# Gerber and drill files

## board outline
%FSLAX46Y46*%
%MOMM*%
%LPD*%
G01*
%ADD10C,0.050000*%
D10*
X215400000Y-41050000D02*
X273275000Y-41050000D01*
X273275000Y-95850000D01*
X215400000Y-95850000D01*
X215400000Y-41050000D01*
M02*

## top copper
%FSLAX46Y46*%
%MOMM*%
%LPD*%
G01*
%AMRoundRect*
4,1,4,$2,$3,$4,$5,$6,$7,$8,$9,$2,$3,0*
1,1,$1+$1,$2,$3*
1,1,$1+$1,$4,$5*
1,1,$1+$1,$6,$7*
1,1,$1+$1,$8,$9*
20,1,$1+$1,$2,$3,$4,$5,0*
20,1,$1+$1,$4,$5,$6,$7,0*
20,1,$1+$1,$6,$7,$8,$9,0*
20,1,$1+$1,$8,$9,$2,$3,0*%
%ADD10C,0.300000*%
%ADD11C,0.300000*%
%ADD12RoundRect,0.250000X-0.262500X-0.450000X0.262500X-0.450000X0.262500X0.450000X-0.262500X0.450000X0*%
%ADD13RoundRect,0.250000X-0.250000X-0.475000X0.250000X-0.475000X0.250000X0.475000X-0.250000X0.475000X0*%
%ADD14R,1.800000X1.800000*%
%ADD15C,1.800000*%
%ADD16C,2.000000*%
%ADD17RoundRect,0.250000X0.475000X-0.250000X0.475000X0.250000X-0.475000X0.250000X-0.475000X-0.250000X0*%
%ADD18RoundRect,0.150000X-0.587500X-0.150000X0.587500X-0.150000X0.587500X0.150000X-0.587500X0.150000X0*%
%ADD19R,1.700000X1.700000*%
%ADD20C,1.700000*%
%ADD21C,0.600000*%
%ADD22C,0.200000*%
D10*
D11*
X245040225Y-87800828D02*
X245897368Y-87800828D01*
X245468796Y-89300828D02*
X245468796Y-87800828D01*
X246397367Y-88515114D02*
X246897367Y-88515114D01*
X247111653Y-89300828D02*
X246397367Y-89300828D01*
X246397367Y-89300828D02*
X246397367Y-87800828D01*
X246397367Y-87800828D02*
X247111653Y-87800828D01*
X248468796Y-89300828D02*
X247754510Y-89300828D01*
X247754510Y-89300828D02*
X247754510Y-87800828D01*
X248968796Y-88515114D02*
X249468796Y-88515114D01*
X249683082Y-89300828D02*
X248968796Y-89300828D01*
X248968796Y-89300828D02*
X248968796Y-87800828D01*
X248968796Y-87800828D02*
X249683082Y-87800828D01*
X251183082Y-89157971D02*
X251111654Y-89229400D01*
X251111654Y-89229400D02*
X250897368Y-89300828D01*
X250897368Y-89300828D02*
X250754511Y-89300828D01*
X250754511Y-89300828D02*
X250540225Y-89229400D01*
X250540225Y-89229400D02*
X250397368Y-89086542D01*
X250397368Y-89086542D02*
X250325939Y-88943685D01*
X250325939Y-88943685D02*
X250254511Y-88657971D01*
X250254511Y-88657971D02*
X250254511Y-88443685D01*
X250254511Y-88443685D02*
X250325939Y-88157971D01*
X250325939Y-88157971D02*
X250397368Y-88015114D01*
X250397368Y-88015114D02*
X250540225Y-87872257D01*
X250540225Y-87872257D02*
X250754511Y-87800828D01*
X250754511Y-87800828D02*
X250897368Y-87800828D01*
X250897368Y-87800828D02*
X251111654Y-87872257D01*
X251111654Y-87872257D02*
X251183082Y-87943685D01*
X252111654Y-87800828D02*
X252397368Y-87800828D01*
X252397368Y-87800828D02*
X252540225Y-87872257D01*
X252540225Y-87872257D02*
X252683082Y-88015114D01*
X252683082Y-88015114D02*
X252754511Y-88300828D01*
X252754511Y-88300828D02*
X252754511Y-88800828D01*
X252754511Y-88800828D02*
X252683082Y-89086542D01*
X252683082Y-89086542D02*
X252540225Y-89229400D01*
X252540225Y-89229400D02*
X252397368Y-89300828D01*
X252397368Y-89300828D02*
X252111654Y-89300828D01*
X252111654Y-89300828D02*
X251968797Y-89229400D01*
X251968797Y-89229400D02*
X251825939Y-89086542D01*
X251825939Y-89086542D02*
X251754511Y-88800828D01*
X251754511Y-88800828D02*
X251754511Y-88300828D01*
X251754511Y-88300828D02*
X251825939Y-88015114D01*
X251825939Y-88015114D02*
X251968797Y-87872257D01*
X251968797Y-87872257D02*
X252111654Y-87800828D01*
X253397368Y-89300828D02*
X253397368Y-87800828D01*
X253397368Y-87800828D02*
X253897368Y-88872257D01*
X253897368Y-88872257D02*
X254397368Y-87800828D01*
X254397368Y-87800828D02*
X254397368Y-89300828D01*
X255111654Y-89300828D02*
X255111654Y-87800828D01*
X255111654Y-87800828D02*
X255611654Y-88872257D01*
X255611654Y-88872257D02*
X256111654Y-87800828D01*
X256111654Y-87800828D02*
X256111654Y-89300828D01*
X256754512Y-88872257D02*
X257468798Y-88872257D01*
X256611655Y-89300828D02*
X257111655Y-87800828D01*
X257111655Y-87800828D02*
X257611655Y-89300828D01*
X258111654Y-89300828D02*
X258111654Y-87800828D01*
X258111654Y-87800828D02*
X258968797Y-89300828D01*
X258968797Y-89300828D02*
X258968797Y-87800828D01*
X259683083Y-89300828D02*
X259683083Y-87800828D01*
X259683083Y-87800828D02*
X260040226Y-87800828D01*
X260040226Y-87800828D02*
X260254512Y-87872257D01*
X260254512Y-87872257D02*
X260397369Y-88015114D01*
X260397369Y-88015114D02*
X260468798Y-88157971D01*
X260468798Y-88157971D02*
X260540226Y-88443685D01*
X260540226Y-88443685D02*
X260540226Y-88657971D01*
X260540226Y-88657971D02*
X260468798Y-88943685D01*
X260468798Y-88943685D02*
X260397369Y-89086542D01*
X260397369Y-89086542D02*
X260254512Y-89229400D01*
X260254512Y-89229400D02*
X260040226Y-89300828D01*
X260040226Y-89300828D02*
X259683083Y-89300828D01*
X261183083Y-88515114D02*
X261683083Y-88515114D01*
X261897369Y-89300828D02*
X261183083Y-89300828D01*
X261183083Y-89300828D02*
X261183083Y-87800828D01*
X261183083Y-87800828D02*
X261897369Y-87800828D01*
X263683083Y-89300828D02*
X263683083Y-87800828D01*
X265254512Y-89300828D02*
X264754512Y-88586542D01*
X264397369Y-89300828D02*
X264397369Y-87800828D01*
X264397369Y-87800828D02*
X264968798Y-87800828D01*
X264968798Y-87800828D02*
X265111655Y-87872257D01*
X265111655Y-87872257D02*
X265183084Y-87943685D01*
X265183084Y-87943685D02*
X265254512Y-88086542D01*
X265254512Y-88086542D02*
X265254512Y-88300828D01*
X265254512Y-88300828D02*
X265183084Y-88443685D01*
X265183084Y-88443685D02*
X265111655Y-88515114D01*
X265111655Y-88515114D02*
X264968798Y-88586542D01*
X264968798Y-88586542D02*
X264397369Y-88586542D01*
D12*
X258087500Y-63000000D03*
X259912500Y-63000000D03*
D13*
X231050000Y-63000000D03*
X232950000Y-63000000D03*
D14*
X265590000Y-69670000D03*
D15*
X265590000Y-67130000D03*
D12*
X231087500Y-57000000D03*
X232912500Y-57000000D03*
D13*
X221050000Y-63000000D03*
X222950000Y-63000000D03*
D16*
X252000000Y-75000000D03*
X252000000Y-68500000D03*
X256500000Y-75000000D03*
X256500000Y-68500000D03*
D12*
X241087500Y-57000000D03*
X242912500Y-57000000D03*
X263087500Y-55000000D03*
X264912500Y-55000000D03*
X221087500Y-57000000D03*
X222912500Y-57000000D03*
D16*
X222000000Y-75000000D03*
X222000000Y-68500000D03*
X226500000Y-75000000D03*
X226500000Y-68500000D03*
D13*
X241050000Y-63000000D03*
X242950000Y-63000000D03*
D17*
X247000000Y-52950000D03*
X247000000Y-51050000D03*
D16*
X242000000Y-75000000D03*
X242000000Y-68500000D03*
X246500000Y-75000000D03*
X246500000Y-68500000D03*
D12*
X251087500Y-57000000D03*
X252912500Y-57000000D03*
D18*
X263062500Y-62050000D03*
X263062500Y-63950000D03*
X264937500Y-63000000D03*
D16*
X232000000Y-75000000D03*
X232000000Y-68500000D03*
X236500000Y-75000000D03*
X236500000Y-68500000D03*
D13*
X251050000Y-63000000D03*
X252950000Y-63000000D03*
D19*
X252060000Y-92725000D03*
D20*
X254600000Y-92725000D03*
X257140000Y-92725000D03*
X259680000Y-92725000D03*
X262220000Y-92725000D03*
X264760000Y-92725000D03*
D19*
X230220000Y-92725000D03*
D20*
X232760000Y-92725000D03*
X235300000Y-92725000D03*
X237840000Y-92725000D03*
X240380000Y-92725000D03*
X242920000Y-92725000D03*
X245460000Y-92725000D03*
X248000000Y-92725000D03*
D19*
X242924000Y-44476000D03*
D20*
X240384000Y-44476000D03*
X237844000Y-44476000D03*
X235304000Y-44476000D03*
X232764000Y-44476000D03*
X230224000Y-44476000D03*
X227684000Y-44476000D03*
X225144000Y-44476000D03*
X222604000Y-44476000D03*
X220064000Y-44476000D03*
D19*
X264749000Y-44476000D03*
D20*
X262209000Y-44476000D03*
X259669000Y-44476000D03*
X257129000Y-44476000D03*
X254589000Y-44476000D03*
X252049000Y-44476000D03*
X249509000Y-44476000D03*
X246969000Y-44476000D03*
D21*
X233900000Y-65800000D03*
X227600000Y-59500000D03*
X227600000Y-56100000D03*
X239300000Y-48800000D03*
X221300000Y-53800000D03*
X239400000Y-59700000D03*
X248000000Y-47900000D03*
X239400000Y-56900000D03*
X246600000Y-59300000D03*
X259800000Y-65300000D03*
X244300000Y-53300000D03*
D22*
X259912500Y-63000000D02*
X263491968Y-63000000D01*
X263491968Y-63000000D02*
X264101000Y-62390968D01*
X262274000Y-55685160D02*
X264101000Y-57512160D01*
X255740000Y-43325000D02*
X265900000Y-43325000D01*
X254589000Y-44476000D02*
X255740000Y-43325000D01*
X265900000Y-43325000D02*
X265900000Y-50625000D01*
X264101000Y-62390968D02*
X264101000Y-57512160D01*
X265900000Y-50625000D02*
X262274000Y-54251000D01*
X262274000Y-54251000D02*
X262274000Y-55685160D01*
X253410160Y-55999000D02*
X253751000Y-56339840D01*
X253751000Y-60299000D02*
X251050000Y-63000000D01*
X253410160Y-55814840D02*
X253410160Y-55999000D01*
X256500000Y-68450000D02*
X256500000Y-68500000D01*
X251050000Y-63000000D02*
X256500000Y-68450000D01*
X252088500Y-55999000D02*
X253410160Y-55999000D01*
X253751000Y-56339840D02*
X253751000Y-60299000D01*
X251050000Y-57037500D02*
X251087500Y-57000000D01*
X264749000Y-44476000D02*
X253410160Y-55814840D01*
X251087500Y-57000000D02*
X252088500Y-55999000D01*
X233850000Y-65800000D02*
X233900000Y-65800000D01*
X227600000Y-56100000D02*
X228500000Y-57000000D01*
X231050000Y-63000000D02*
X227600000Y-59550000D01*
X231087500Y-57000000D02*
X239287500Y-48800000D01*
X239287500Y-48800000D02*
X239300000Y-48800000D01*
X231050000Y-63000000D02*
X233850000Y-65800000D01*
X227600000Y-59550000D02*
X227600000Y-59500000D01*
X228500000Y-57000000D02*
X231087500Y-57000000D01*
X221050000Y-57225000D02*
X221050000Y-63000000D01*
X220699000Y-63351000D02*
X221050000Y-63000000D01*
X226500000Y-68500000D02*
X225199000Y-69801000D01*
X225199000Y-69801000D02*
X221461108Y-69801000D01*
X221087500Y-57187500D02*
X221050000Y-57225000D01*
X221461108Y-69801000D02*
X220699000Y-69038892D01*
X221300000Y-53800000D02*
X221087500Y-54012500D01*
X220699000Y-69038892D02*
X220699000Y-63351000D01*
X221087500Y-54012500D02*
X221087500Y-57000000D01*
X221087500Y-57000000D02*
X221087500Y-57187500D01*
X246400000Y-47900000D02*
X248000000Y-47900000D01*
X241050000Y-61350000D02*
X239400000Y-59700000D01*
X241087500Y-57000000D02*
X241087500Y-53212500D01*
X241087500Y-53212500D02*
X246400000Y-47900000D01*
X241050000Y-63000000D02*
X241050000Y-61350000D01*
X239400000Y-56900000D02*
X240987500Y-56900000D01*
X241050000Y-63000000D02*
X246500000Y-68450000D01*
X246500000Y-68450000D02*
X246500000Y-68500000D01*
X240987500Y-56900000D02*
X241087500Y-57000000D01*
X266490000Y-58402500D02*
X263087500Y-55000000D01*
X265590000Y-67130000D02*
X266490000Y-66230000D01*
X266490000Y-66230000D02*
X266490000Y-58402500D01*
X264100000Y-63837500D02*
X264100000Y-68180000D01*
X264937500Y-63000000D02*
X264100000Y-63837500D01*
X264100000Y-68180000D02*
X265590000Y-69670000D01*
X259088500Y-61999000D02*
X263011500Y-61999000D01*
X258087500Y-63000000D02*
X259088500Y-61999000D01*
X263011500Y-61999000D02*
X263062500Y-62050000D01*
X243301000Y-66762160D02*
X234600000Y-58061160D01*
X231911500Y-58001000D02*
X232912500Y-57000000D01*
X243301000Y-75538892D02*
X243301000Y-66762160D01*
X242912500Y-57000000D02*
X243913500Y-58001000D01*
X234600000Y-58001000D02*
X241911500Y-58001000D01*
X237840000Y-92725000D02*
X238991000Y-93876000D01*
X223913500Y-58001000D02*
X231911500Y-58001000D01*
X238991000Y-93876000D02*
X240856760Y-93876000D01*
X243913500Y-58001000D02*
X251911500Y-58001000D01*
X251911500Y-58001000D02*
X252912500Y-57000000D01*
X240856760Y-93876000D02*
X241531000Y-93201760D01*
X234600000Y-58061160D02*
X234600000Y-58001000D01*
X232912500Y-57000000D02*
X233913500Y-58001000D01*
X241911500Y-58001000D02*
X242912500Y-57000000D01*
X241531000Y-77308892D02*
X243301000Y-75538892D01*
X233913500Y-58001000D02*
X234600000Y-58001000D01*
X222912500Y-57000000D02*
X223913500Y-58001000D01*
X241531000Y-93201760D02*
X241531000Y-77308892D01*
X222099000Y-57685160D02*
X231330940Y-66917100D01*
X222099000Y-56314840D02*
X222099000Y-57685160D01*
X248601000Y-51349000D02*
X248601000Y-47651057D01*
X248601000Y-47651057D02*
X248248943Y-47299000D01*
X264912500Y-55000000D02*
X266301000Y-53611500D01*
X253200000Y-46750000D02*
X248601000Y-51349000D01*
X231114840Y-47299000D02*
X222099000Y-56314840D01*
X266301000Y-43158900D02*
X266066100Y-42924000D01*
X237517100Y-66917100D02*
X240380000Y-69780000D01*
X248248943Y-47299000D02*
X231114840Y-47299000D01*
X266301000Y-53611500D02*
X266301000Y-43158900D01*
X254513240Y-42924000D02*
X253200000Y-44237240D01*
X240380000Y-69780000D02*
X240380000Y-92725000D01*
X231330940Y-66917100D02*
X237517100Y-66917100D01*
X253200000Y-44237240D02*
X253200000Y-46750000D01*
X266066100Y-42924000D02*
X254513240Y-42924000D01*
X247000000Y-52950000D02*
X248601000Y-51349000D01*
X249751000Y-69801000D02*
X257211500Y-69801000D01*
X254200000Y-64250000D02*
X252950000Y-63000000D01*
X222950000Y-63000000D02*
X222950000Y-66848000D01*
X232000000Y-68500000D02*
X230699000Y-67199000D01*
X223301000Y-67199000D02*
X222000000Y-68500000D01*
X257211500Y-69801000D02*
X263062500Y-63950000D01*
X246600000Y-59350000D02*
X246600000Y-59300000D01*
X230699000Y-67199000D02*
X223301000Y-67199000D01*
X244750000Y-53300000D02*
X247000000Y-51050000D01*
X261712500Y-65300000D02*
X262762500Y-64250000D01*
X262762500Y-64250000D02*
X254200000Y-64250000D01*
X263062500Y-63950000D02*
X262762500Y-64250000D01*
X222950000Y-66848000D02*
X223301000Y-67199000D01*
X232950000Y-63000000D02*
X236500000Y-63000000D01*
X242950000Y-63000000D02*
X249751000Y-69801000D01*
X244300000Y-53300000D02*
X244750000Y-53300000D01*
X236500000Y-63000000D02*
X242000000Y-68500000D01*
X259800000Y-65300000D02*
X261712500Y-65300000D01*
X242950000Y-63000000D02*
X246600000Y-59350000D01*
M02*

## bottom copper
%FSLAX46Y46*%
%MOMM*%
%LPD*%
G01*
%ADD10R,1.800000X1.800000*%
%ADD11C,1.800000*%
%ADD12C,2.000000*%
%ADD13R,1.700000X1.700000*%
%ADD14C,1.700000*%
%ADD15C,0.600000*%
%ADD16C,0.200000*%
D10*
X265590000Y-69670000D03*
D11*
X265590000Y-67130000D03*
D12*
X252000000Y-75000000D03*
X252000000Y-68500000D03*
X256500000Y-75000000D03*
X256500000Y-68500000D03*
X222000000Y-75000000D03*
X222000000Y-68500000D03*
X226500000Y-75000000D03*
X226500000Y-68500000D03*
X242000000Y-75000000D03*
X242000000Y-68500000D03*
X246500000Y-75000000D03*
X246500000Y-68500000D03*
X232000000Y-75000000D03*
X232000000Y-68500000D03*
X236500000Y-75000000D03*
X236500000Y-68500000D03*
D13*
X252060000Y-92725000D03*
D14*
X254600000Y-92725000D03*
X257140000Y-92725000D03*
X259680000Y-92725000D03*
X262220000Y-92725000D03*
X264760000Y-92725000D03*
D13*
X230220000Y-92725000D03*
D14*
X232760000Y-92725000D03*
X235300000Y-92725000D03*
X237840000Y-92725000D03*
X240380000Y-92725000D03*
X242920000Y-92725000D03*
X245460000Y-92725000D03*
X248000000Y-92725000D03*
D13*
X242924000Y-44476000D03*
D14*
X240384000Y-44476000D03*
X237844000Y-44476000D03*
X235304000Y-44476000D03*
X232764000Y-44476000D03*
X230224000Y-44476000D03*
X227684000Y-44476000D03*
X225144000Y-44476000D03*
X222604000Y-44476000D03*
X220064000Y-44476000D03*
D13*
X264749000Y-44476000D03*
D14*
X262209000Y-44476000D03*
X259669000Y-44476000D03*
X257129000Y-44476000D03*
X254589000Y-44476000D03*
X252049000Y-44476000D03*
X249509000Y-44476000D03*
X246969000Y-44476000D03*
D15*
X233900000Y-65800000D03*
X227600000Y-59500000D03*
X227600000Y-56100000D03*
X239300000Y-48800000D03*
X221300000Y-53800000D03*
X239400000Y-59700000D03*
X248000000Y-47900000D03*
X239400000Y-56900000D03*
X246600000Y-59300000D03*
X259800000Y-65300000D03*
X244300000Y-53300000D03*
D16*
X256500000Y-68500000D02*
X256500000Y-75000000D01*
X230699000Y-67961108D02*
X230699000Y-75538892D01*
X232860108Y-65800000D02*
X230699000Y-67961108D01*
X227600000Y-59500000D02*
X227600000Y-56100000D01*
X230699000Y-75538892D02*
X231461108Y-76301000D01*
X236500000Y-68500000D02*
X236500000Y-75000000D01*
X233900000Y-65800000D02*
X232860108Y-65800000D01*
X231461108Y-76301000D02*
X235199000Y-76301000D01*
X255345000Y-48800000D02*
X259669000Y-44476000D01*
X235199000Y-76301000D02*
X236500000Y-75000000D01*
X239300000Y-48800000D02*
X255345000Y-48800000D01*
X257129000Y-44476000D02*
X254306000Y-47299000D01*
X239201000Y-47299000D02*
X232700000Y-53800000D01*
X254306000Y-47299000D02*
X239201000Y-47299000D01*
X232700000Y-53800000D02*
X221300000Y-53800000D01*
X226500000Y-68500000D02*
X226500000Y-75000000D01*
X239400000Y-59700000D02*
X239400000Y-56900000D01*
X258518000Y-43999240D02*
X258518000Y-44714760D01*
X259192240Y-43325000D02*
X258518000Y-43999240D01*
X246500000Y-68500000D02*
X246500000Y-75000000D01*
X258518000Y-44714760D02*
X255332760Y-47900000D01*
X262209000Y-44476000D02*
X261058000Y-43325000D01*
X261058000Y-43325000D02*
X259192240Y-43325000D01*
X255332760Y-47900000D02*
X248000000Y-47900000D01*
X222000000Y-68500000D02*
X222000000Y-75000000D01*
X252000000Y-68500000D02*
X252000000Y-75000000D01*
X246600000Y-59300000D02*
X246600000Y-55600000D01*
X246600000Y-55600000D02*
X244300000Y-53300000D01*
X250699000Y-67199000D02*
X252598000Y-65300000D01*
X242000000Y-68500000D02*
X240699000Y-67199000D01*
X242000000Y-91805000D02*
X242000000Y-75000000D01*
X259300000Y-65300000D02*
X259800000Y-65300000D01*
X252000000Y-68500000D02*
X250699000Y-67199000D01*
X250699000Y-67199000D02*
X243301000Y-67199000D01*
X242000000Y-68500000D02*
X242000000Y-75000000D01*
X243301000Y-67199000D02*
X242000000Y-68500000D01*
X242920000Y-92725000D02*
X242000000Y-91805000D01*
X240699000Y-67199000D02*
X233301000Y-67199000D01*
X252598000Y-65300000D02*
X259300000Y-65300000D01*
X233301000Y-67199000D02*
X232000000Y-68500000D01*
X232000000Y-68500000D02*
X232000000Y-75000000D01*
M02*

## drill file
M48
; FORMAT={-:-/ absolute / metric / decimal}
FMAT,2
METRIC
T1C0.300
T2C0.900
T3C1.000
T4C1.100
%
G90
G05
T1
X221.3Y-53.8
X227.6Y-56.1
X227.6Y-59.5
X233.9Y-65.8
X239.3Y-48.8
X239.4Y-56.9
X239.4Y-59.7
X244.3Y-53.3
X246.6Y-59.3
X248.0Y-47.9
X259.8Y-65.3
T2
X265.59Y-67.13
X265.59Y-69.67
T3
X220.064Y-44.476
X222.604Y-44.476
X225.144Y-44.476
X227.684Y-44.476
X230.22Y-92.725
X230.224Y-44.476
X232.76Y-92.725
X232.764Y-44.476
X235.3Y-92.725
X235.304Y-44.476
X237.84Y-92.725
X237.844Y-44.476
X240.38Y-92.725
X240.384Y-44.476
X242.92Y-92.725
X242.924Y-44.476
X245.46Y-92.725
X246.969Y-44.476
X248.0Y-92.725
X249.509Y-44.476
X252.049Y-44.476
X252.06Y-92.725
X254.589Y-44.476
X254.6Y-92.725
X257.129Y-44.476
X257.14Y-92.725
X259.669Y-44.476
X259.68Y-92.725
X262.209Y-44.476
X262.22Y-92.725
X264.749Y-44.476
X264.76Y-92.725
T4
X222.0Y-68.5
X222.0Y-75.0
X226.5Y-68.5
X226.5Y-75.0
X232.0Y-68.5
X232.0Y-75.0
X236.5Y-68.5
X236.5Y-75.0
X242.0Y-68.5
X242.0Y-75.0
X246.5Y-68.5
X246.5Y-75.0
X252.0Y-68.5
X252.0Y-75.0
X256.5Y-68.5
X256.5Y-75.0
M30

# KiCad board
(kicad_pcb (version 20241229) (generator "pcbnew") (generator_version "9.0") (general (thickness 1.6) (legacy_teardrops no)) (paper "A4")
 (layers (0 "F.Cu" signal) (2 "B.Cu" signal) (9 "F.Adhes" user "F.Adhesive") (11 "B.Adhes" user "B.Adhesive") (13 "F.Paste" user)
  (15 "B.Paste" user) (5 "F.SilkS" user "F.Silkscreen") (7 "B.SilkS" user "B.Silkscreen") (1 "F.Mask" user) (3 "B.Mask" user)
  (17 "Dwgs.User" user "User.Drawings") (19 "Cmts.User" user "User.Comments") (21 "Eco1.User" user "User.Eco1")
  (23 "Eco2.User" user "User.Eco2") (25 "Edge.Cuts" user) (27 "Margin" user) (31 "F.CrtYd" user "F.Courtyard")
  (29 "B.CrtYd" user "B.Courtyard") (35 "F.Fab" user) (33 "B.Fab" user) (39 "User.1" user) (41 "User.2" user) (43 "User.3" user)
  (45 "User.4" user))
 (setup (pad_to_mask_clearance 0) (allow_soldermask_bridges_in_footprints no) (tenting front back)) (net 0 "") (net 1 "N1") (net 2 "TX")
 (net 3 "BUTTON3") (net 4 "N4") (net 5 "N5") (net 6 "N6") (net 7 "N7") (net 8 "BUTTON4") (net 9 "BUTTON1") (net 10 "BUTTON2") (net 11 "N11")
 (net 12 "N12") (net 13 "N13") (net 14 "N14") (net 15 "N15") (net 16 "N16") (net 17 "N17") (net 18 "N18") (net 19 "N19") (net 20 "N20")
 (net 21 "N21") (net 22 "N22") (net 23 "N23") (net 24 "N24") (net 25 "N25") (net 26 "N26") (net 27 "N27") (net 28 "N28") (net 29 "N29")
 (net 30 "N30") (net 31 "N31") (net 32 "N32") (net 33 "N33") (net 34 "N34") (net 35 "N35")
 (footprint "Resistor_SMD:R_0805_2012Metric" (layer "F.Cu") (at 259 63)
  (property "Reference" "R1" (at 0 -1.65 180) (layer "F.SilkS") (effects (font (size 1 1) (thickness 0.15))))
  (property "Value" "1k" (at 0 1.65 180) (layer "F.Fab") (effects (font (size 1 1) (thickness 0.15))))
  (pad "1" smd roundrect (at -0.9125 0) (size 1.025 1.4) (layers "F.Cu" "F.Mask" "F.Paste") (roundrect_rratio 0.243902) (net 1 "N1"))
  (pad "2" smd roundrect (at 0.9125 0) (size 1.025 1.4) (layers "F.Cu" "F.Mask" "F.Paste") (roundrect_rratio 0.243902) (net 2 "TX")))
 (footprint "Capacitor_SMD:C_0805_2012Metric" (layer "F.Cu") (at 232 63)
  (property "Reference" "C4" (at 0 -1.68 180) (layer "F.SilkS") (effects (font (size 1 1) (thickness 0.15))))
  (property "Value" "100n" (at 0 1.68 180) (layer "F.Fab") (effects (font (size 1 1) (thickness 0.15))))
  (pad "1" smd roundrect (at -0.95 0) (size 1 1.45) (layers "F.Cu" "F.Mask" "F.Paste") (roundrect_rratio 0.25) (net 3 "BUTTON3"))
  (pad "2" smd roundrect (at 0.95 0) (size 1 1.45) (layers "F.Cu" "F.Mask" "F.Paste") (roundrect_rratio 0.25) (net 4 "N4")))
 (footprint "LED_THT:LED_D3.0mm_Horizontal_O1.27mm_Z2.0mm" (layer "F.Cu") (at 265.59 69.67 90)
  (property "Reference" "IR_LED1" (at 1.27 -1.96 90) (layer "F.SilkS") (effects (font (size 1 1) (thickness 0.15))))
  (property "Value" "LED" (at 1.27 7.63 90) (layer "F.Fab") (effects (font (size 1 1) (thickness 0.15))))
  (pad "1" thru_hole rect (at 0 0 90) (size 1.8 1.8) (drill 0.9) (layers "*.Cu" "*.Mask") (remove_unused_layers no) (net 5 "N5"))
  (pad "2" thru_hole circle (at 2.54 0 90) (size 1.8 1.8) (drill 0.9) (layers "*.Cu" "*.Mask") (remove_unused_layers no) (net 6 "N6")))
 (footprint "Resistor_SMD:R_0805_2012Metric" (layer "F.Cu") (at 232 57)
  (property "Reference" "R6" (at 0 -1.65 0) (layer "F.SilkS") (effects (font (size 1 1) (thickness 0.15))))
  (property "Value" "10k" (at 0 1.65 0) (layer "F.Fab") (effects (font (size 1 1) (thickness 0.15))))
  (pad "1" smd roundrect (at -0.9125 0) (size 1.025 1.4) (layers "F.Cu" "F.Mask" "F.Paste") (roundrect_rratio 0.243902) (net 3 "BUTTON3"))
  (pad "2" smd roundrect (at 0.9125 0) (size 1.025 1.4) (layers "F.Cu" "F.Mask" "F.Paste") (roundrect_rratio 0.243902) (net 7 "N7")))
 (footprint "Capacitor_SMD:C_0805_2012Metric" (layer "F.Cu") (at 222 63)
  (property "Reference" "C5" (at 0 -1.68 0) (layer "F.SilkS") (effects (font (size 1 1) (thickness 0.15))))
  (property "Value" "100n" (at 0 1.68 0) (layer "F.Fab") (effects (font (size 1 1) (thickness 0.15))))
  (pad "1" smd roundrect (at -0.95 0) (size 1 1.45) (layers "F.Cu" "F.Mask" "F.Paste") (roundrect_rratio 0.25) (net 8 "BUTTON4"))
  (pad "2" smd roundrect (at 0.95 0) (size 1 1.45) (layers "F.Cu" "F.Mask" "F.Paste") (roundrect_rratio 0.25) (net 4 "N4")))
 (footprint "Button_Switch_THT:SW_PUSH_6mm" (layer "F.Cu") (at 252 75 90)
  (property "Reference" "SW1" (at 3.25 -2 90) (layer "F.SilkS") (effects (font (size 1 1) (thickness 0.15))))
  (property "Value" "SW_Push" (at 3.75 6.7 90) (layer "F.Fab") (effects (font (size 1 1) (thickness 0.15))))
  (pad "1" thru_hole circle (at 0 0 180) (size 2 2) (drill 1.1) (layers "*.Cu" "*.Mask") (remove_unused_layers no) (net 4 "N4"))
  (pad "1" thru_hole circle (at 6.5 0 180) (size 2 2) (drill 1.1) (layers "*.Cu" "*.Mask") (remove_unused_layers no) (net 4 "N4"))
  (pad "2" thru_hole circle (at 0 4.5 180) (size 2 2) (drill 1.1) (layers "*.Cu" "*.Mask") (remove_unused_layers no) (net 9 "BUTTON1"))
  (pad "2" thru_hole circle (at 6.5 4.5 180) (size 2 2) (drill 1.1) (layers "*.Cu" "*.Mask") (remove_unused_layers no) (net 9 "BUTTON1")))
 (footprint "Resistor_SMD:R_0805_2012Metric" (layer "F.Cu") (at 242 57)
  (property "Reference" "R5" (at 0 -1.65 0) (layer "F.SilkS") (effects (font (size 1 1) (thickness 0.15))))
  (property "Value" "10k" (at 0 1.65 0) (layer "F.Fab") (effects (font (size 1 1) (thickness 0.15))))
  (pad "1" smd roundrect (at -0.9125 0) (size 1.025 1.4) (layers "F.Cu" "F.Mask" "F.Paste") (roundrect_rratio 0.243902) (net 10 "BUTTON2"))
  (pad "2" smd roundrect (at 0.9125 0) (size 1.025 1.4) (layers "F.Cu" "F.Mask" "F.Paste") (roundrect_rratio 0.243902) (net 7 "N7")))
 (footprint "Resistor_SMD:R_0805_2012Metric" (layer "F.Cu") (at 264 55)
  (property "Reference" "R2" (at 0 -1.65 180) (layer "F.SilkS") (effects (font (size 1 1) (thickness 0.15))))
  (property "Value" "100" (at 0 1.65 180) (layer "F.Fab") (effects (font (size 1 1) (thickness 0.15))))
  (pad "1" smd roundrect (at -0.9125 0) (size 1.025 1.4) (layers "F.Cu" "F.Mask" "F.Paste") (roundrect_rratio 0.243902) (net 6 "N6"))
  (pad "2" smd roundrect (at 0.9125 0) (size 1.025 1.4) (layers "F.Cu" "F.Mask" "F.Paste") (roundrect_rratio 0.243902) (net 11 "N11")))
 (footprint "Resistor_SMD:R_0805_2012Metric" (layer "F.Cu") (at 222 57)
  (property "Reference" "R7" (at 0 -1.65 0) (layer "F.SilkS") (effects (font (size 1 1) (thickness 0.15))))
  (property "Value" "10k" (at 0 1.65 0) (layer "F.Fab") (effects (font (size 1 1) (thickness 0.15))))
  (pad "1" smd roundrect (at -0.9125 0) (size 1.025 1.4) (layers "F.Cu" "F.Mask" "F.Paste") (roundrect_rratio 0.243902) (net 8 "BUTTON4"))
  (pad "2" smd roundrect (at 0.9125 0) (size 1.025 1.4) (layers "F.Cu" "F.Mask" "F.Paste") (roundrect_rratio 0.243902) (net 7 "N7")))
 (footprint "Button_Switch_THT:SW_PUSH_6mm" (layer "F.Cu") (at 222 75 90)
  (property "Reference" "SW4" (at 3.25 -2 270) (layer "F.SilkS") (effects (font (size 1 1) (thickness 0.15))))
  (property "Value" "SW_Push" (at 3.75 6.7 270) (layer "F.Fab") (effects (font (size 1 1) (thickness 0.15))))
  (pad "1" thru_hole circle (at 0 0 180) (size 2 2) (drill 1.1) (layers "*.Cu" "*.Mask") (remove_unused_layers no) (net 4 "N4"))
  (pad "1" thru_hole circle (at 6.5 0 180) (size 2 2) (drill 1.1) (layers "*.Cu" "*.Mask") (remove_unused_layers no) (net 4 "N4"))
  (pad "2" thru_hole circle (at 0 4.5 180) (size 2 2) (drill 1.1) (layers "*.Cu" "*.Mask") (remove_unused_layers no) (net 8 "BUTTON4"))
  (pad "2" thru_hole circle (at 6.5 4.5 180) (size 2 2) (drill 1.1) (layers "*.Cu" "*.Mask") (remove_unused_layers no) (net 8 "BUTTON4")))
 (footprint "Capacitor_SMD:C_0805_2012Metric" (layer "F.Cu") (at 242 63)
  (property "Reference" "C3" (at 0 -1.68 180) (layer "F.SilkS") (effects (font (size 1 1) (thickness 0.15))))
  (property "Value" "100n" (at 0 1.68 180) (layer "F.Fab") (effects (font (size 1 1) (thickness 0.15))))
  (pad "1" smd roundrect (at -0.95 0) (size 1 1.45) (layers "F.Cu" "F.Mask" "F.Paste") (roundrect_rratio 0.25) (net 10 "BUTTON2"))
  (pad "2" smd roundrect (at 0.95 0) (size 1 1.45) (layers "F.Cu" "F.Mask" "F.Paste") (roundrect_rratio 0.25) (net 4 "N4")))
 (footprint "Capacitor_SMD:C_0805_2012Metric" (layer "F.Cu") (at 247 52 90)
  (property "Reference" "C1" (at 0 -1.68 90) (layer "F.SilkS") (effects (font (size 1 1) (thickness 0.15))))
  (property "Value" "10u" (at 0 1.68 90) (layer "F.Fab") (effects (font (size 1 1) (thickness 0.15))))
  (pad "1" smd roundrect (at -0.95 0 90) (size 1 1.45) (layers "F.Cu" "F.Mask" "F.Paste") (roundrect_rratio 0.25) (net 11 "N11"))
  (pad "2" smd roundrect (at 0.95 0 90) (size 1 1.45) (layers "F.Cu" "F.Mask" "F.Paste") (roundrect_rratio 0.25) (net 4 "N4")))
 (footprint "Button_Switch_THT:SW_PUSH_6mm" (layer "F.Cu") (at 242 75 90)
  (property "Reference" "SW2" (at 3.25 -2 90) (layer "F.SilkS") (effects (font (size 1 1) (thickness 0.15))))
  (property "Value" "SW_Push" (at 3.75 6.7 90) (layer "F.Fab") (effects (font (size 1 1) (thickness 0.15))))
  (pad "1" thru_hole circle (at 0 0 180) (size 2 2) (drill 1.1) (layers "*.Cu" "*.Mask") (remove_unused_layers no) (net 4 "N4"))
  (pad "1" thru_hole circle (at 6.5 0 180) (size 2 2) (drill 1.1) (layers "*.Cu" "*.Mask") (remove_unused_layers no) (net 4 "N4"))
  (pad "2" thru_hole circle (at 0 4.5 180) (size 2 2) (drill 1.1) (layers "*.Cu" "*.Mask") (remove_unused_layers no) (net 10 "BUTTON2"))
  (pad "2" thru_hole circle (at 6.5 4.5 180) (size 2 2) (drill 1.1) (layers "*.Cu" "*.Mask") (remove_unused_layers no) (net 10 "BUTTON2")))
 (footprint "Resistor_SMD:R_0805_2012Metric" (layer "F.Cu") (at 252 57)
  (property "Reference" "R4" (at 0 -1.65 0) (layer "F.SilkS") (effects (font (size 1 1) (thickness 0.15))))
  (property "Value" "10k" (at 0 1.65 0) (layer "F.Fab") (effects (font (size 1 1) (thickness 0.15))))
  (pad "1" smd roundrect (at -0.9125 0) (size 1.025 1.4) (layers "F.Cu" "F.Mask" "F.Paste") (roundrect_rratio 0.243902) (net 9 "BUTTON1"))
  (pad "2" smd roundrect (at 0.9125 0) (size 1.025 1.4) (layers "F.Cu" "F.Mask" "F.Paste") (roundrect_rratio 0.243902) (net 7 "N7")))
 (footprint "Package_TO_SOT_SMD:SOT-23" (layer "F.Cu") (at 264 63)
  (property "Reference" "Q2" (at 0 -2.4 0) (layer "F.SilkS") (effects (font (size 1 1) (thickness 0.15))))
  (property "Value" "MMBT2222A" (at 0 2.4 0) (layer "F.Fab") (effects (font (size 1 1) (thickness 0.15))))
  (pad "1" smd roundrect (at -0.9375 -0.95) (size 1.475 0.6) (layers "F.Cu" "F.Mask" "F.Paste") (roundrect_rratio 0.25) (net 1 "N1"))
  (pad "2" smd roundrect (at -0.9375 0.95) (size 1.475 0.6) (layers "F.Cu" "F.Mask" "F.Paste") (roundrect_rratio 0.25) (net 4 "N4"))
  (pad "3" smd roundrect (at 0.9375 0) (size 1.475 0.6) (layers "F.Cu" "F.Mask" "F.Paste") (roundrect_rratio 0.25) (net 5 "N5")))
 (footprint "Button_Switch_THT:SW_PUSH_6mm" (layer "F.Cu") (at 232 75 90)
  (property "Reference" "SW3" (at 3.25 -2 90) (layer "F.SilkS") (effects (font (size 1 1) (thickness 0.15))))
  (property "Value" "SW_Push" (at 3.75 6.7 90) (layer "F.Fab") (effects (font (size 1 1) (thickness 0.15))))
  (pad "1" thru_hole circle (at 0 0 180) (size 2 2) (drill 1.1) (layers "*.Cu" "*.Mask") (remove_unused_layers no) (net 4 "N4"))
  (pad "1" thru_hole circle (at 6.5 0 180) (size 2 2) (drill 1.1) (layers "*.Cu" "*.Mask") (remove_unused_layers no) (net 4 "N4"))
  (pad "2" thru_hole circle (at 0 4.5 180) (size 2 2) (drill 1.1) (layers "*.Cu" "*.Mask") (remove_unused_layers no) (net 3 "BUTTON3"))
  (pad "2" thru_hole circle (at 6.5 4.5 180) (size 2 2) (drill 1.1) (layers "*.Cu" "*.Mask") (remove_unused_layers no) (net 3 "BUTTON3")))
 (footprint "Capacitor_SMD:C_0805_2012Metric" (layer "F.Cu") (at 252 63)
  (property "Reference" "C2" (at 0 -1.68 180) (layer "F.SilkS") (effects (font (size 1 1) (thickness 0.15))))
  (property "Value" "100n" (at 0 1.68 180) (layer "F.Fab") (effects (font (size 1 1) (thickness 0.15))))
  (pad "1" smd roundrect (at -0.95 0) (size 1 1.45) (layers "F.Cu" "F.Mask" "F.Paste") (roundrect_rratio 0.25) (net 9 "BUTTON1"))
  (pad "2" smd roundrect (at 0.95 0) (size 1 1.45) (layers "F.Cu" "F.Mask" "F.Paste") (roundrect_rratio 0.25) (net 4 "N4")))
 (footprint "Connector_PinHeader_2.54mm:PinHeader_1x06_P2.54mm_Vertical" (layer "B.Cu") (at 252.06 92.725 -90)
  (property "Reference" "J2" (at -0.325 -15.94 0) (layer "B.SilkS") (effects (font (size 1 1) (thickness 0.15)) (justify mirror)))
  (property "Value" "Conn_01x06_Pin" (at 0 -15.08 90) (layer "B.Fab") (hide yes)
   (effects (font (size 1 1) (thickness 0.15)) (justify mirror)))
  (pad "1" thru_hole rect (at 0 0 270) (size 1.7 1.7) (drill 1) (layers "*.Cu" "*.Mask") (remove_unused_layers no) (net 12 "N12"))
  (pad "2" thru_hole circle (at 0 -2.54 270) (size 1.7 1.7) (drill 1) (layers "*.Cu" "*.Mask") (remove_unused_layers no) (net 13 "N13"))
  (pad "3" thru_hole circle (at 0 -5.08 270) (size 1.7 1.7) (drill 1) (layers "*.Cu" "*.Mask") (remove_unused_layers no) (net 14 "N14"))
  (pad "4" thru_hole circle (at 0 -7.62 270) (size 1.7 1.7) (drill 1) (layers "*.Cu" "*.Mask") (remove_unused_layers no) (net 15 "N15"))
  (pad "5" thru_hole circle (at 0 -10.16 270) (size 1.7 1.7) (drill 1) (layers "*.Cu" "*.Mask") (remove_unused_layers no) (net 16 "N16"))
  (pad "6" thru_hole circle (at 0 -12.7 270) (size 1.7 1.7) (drill 1) (layers "*.Cu" "*.Mask") (remove_unused_layers no) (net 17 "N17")))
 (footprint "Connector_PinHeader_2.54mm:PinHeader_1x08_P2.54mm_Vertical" (layer "B.Cu") (at 230.22 92.725 -90)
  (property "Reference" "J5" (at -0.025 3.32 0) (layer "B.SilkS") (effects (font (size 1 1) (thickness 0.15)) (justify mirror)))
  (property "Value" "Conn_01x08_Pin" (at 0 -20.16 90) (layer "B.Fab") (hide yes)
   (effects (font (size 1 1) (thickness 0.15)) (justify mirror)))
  (pad "1" thru_hole rect (at 0 0 270) (size 1.7 1.7) (drill 1) (layers "*.Cu" "*.Mask") (remove_unused_layers no) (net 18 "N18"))
  (pad "2" thru_hole circle (at 0 -2.54 270) (size 1.7 1.7) (drill 1) (layers "*.Cu" "*.Mask") (remove_unused_layers no) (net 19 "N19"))
  (pad "3" thru_hole circle (at 0 -5.08 270) (size 1.7 1.7) (drill 1) (layers "*.Cu" "*.Mask") (remove_unused_layers no) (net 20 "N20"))
  (pad "4" thru_hole circle (at 0 -7.62 270) (size 1.7 1.7) (drill 1) (layers "*.Cu" "*.Mask") (remove_unused_layers no) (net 7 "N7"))
  (pad "5" thru_hole circle (at 0 -10.16 270) (size 1.7 1.7) (drill 1) (layers "*.Cu" "*.Mask") (remove_unused_layers no) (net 11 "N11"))
  (pad "6" thru_hole circle (at 0 -12.7 270) (size 1.7 1.7) (drill 1) (layers "*.Cu" "*.Mask") (remove_unused_layers no) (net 4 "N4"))
  (pad "7" thru_hole circle (at 0 -15.24 270) (size 1.7 1.7) (drill 1) (layers "*.Cu" "*.Mask") (remove_unused_layers no) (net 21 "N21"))
  (pad "8" thru_hole circle (at 0 -17.78 270) (size 1.7 1.7) (drill 1) (layers "*.Cu" "*.Mask") (remove_unused_layers no) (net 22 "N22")))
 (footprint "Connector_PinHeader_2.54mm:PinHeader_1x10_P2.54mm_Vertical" (layer "B.Cu") (at 242.924 44.476 90)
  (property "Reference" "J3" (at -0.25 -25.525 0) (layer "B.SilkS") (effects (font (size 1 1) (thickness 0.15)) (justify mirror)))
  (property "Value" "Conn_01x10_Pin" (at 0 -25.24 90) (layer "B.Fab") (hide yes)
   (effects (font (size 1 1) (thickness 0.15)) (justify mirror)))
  (pad "1" thru_hole rect (at 0 0 90) (size 1.7 1.7) (drill 1) (layers "*.Cu" "*.Mask") (remove_unused_layers no) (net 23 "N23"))
  (pad "2" thru_hole circle (at 0 -2.54 90) (size 1.7 1.7) (drill 1) (layers "*.Cu" "*.Mask") (remove_unused_layers no) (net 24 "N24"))
  (pad "3" thru_hole circle (at 0 -5.08 90) (size 1.7 1.7) (drill 1) (layers "*.Cu" "*.Mask") (remove_unused_layers no) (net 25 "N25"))
  (pad "4" thru_hole circle (at 0 -7.62 90) (size 1.7 1.7) (drill 1) (layers "*.Cu" "*.Mask") (remove_unused_layers no) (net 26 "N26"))
  (pad "5" thru_hole circle (at 0 -10.16 90) (size 1.7 1.7) (drill 1) (layers "*.Cu" "*.Mask") (remove_unused_layers no) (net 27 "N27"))
  (pad "6" thru_hole circle (at 0 -12.7 90) (size 1.7 1.7) (drill 1) (layers "*.Cu" "*.Mask") (remove_unused_layers no) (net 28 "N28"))
  (pad "7" thru_hole circle (at 0 -15.24 90) (size 1.7 1.7) (drill 1) (layers "*.Cu" "*.Mask") (remove_unused_layers no) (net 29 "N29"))
  (pad "8" thru_hole circle (at 0 -17.78 90) (size 1.7 1.7) (drill 1) (layers "*.Cu" "*.Mask") (remove_unused_layers no) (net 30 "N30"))
  (pad "9" thru_hole circle (at 0 -20.32 90) (size 1.7 1.7) (drill 1) (layers "*.Cu" "*.Mask") (remove_unused_layers no) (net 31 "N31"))
  (pad "10" thru_hole circle (at 0 -22.86 90) (size 1.7 1.7) (drill 1) (layers "*.Cu" "*.Mask") (remove_unused_layers no) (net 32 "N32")))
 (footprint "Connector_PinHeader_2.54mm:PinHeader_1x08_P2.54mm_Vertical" (layer "B.Cu") (at 264.749 44.476 90)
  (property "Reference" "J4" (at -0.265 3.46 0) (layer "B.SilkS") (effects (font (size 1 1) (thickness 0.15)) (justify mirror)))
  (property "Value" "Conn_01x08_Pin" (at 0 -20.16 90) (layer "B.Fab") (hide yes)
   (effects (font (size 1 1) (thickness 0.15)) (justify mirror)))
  (pad "1" thru_hole rect (at 0 0 90) (size 1.7 1.7) (drill 1) (layers "*.Cu" "*.Mask") (remove_unused_layers no) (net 9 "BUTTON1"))
  (pad "2" thru_hole circle (at 0 -2.54 90) (size 1.7 1.7) (drill 1) (layers "*.Cu" "*.Mask") (remove_unused_layers no) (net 10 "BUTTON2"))
  (pad "3" thru_hole circle (at 0 -5.08 90) (size 1.7 1.7) (drill 1) (layers "*.Cu" "*.Mask") (remove_unused_layers no) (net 3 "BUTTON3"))
  (pad "4" thru_hole circle (at 0 -7.62 90) (size 1.7 1.7) (drill 1) (layers "*.Cu" "*.Mask") (remove_unused_layers no) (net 8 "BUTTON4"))
  (pad "5" thru_hole circle (at 0 -10.16 90) (size 1.7 1.7) (drill 1) (layers "*.Cu" "*.Mask") (remove_unused_layers no) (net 2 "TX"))
  (pad "6" thru_hole circle (at 0 -12.7 90) (size 1.7 1.7) (drill 1) (layers "*.Cu" "*.Mask") (remove_unused_layers no) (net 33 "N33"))
  (pad "7" thru_hole circle (at 0 -15.24 90) (size 1.7 1.7) (drill 1) (layers "*.Cu" "*.Mask") (remove_unused_layers no) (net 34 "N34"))
  (pad "8" thru_hole circle (at 0 -17.78 90) (size 1.7 1.7) (drill 1) (layers "*.Cu" "*.Mask") (remove_unused_layers no) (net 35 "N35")))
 (gr_rect (start 215.4 41.05) (end 273.275 95.85) (stroke (width 0.05) (type solid)) (fill no) (layer "Edge.Cuts"))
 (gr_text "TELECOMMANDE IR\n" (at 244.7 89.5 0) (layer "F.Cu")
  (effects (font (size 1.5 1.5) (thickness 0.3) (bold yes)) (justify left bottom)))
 (segment (start 259.9125 63) (end 263.491968 63) (width 0.2) (layer "F.Cu") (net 2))
 (segment (start 263.491968 63) (end 264.101 62.390968) (width 0.2) (layer "F.Cu") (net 2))
 (segment (start 262.274 55.68516) (end 264.101 57.51216) (width 0.2) (layer "F.Cu") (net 2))
 (segment (start 255.74 43.325) (end 265.9 43.325) (width 0.2) (layer "F.Cu") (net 2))
 (segment (start 254.589 44.476) (end 255.74 43.325) (width 0.2) (layer "F.Cu") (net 2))
 (segment (start 265.9 43.325) (end 265.9 50.625) (width 0.2) (layer "F.Cu") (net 2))
 (segment (start 264.101 62.390968) (end 264.101 57.51216) (width 0.2) (layer "F.Cu") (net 2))
 (segment (start 265.9 50.625) (end 262.274 54.251) (width 0.2) (layer "F.Cu") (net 2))
 (segment (start 262.274 54.251) (end 262.274 55.68516) (width 0.2) (layer "F.Cu") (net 2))
 (segment (start 253.41016 55.999) (end 253.751 56.33984) (width 0.2) (layer "F.Cu") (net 9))
 (segment (start 253.751 60.299) (end 251.05 63) (width 0.2) (layer "F.Cu") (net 9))
 (segment (start 253.41016 55.81484) (end 253.41016 55.999) (width 0.2) (layer "F.Cu") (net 9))
 (segment (start 256.5 68.45) (end 256.5 68.5) (width 0.2) (layer "F.Cu") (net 9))
 (segment (start 251.05 63) (end 256.5 68.45) (width 0.2) (layer "F.Cu") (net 9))
 (segment (start 252.0885 55.999) (end 253.41016 55.999) (width 0.2) (layer "F.Cu") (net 9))
 (segment (start 253.751 56.33984) (end 253.751 60.299) (width 0.2) (layer "F.Cu") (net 9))
 (segment (start 251.05 57.0375) (end 251.0875 57) (width 0.2) (layer "F.Cu") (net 9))
 (segment (start 264.749 44.476) (end 253.41016 55.81484) (width 0.2) (layer "F.Cu") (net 9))
 (segment (start 251.0875 57) (end 252.0885 55.999) (width 0.2) (layer "F.Cu") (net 9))
 (segment (start 256.5 68.5) (end 256.5 75) (width 0.2) (layer "B.Cu") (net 9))
 (segment (start 233.85 65.8) (end 233.9 65.8) (width 0.2) (layer "F.Cu") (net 3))
 (segment (start 227.6 56.1) (end 228.5 57) (width 0.2) (layer "F.Cu") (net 3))
 (segment (start 231.05 63) (end 227.6 59.55) (width 0.2) (layer "F.Cu") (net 3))
 (segment (start 231.0875 57) (end 239.2875 48.8) (width 0.2) (layer "F.Cu") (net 3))
 (segment (start 239.2875 48.8) (end 239.3 48.8) (width 0.2) (layer "F.Cu") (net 3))
 (segment (start 231.05 63) (end 233.85 65.8) (width 0.2) (layer "F.Cu") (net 3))
 (segment (start 227.6 59.55) (end 227.6 59.5) (width 0.2) (layer "F.Cu") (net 3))
 (segment (start 228.5 57) (end 231.0875 57) (width 0.2) (layer "F.Cu") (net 3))
 (via (at 233.9 65.8) (size 0.6) (drill 0.3) (layers "F.Cu" "B.Cu") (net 3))
 (via (at 227.6 59.5) (size 0.6) (drill 0.3) (layers "F.Cu" "B.Cu") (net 3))
 (via (at 227.6 56.1) (size 0.6) (drill 0.3) (layers "F.Cu" "B.Cu") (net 3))
 (via (at 239.3 48.8) (size 0.6) (drill 0.3) (layers "F.Cu" "B.Cu") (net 3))
 (segment (start 230.699 67.961108) (end 230.699 75.538892) (width 0.2) (layer "B.Cu") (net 3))
 (segment (start 232.860108 65.8) (end 230.699 67.961108) (width 0.2) (layer "B.Cu") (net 3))
 (segment (start 227.6 59.5) (end 227.6 56.1) (width 0.2) (layer "B.Cu") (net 3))
 (segment (start 230.699 75.538892) (end 231.461108 76.301) (width 0.2) (layer "B.Cu") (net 3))
 (segment (start 236.5 68.5) (end 236.5 75) (width 0.2) (layer "B.Cu") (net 3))
 (segment (start 233.9 65.8) (end 232.860108 65.8) (width 0.2) (layer "B.Cu") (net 3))
 (segment (start 231.461108 76.301) (end 235.199 76.301) (width 0.2) (layer "B.Cu") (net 3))
 (segment (start 255.345 48.8) (end 259.669 44.476) (width 0.2) (layer "B.Cu") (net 3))
 (segment (start 235.199 76.301) (end 236.5 75) (width 0.2) (layer "B.Cu") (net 3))
 (segment (start 239.3 48.8) (end 255.345 48.8) (width 0.2) (layer "B.Cu") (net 3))
 (segment (start 221.05 57.225) (end 221.05 63) (width 0.2) (layer "F.Cu") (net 8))
 (segment (start 220.699 63.351) (end 221.05 63) (width 0.2) (layer "F.Cu") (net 8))
 (segment (start 226.5 68.5) (end 225.199 69.801) (width 0.2) (layer "F.Cu") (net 8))
 (segment (start 225.199 69.801) (end 221.461108 69.801) (width 0.2) (layer "F.Cu") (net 8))
 (segment (start 221.0875 57.1875) (end 221.05 57.225) (width 0.2) (layer "F.Cu") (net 8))
 (segment (start 221.461108 69.801) (end 220.699 69.038892) (width 0.2) (layer "F.Cu") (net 8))
 (segment (start 221.3 53.8) (end 221.0875 54.0125) (width 0.2) (layer "F.Cu") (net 8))
 (segment (start 220.699 69.038892) (end 220.699 63.351) (width 0.2) (layer "F.Cu") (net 8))
 (segment (start 221.0875 54.0125) (end 221.0875 57) (width 0.2) (layer "F.Cu") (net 8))
 (segment (start 221.0875 57) (end 221.0875 57.1875) (width 0.2) (layer "F.Cu") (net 8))
 (via (at 221.3 53.8) (size 0.6) (drill 0.3) (layers "F.Cu" "B.Cu") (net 8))
 (segment (start 257.129 44.476) (end 254.306 47.299) (width 0.2) (layer "B.Cu") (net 8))
 (segment (start 239.201 47.299) (end 232.7 53.8) (width 0.2) (layer "B.Cu") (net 8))
 (segment (start 254.306 47.299) (end 239.201 47.299) (width 0.2) (layer "B.Cu") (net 8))
 (segment (start 232.7 53.8) (end 221.3 53.8) (width 0.2) (layer "B.Cu") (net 8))
 (segment (start 226.5 68.5) (end 226.5 75) (width 0.2) (layer "B.Cu") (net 8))
 (segment (start 246.4 47.9) (end 248 47.9) (width 0.2) (layer "F.Cu") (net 10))
 (segment (start 241.05 61.35) (end 239.4 59.7) (width 0.2) (layer "F.Cu") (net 10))
 (segment (start 241.0875 57) (end 241.0875 53.2125) (width 0.2) (layer "F.Cu") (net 10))
 (segment (start 241.0875 53.2125) (end 246.4 47.9) (width 0.2) (layer "F.Cu") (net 10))
 (segment (start 241.05 63) (end 241.05 61.35) (width 0.2) (layer "F.Cu") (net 10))
 (segment (start 239.4 56.9) (end 240.9875 56.9) (width 0.2) (layer "F.Cu") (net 10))
 (segment (start 241.05 63) (end 246.5 68.45) (width 0.2) (layer "F.Cu") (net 10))
 (segment (start 246.5 68.45) (end 246.5 68.5) (width 0.2) (layer "F.Cu") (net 10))
 (segment (start 240.9875 56.9) (end 241.0875 57) (width 0.2) (layer "F.Cu") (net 10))
 (via (at 239.4 59.7) (size 0.6) (drill 0.3) (layers "F.Cu" "B.Cu") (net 10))
 (via (at 248 47.9) (size 0.6) (drill 0.3) (layers "F.Cu" "B.Cu") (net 10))
 (via (at 239.4 56.9) (size 0.6) (drill 0.3) (layers "F.Cu" "B.Cu") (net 10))
 (segment (start 239.4 59.7) (end 239.4 56.9) (width 0.2) (layer "B.Cu") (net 10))
 (segment (start 258.518 43.99924) (end 258.518 44.71476) (width 0.2) (layer "B.Cu") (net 10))
 (segment (start 259.19224 43.325) (end 258.518 43.99924) (width 0.2) (layer "B.Cu") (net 10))
 (segment (start 246.5 68.5) (end 246.5 75) (width 0.2) (layer "B.Cu") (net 10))
 (segment (start 258.518 44.71476) (end 255.33276 47.9) (width 0.2) (layer "B.Cu") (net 10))
 (segment (start 262.209 44.476) (end 261.058 43.325) (width 0.2) (layer "B.Cu") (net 10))
 (segment (start 261.058 43.325) (end 259.19224 43.325) (width 0.2) (layer "B.Cu") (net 10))
 (segment (start 255.33276 47.9) (end 248 47.9) (width 0.2) (layer "B.Cu") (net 10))
 (segment (start 266.49 58.4025) (end 263.0875 55) (width 0.2) (layer "F.Cu") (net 6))
 (segment (start 265.59 67.13) (end 266.49 66.23) (width 0.2) (layer "F.Cu") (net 6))
 (segment (start 266.49 66.23) (end 266.49 58.4025) (width 0.2) (layer "F.Cu") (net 6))
 (segment (start 264.1 63.8375) (end 264.1 68.18) (width 0.2) (layer "F.Cu") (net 5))
 (segment (start 264.9375 63) (end 264.1 63.8375) (width 0.2) (layer "F.Cu") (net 5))
 (segment (start 264.1 68.18) (end 265.59 69.67) (width 0.2) (layer "F.Cu") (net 5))
 (segment (start 259.0885 61.999) (end 263.0115 61.999) (width 0.2) (layer "F.Cu") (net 1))
 (segment (start 258.0875 63) (end 259.0885 61.999) (width 0.2) (layer "F.Cu") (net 1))
 (segment (start 263.0115 61.999) (end 263.0625 62.05) (width 0.2) (layer "F.Cu") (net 1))
 (segment (start 243.301 66.76216) (end 234.6 58.06116) (width 0.2) (layer "F.Cu") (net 7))
 (segment (start 231.9115 58.001) (end 232.9125 57) (width 0.2) (layer "F.Cu") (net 7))
 (segment (start 243.301 75.538892) (end 243.301 66.76216) (width 0.2) (layer "F.Cu") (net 7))
 (segment (start 242.9125 57) (end 243.9135 58.001) (width 0.2) (layer "F.Cu") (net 7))
 (segment (start 234.6 58.001) (end 241.9115 58.001) (width 0.2) (layer "F.Cu") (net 7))
 (segment (start 237.84 92.725) (end 238.991 93.876) (width 0.2) (layer "F.Cu") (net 7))
 (segment (start 223.9135 58.001) (end 231.9115 58.001) (width 0.2) (layer "F.Cu") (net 7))
 (segment (start 238.991 93.876) (end 240.85676 93.876) (width 0.2) (layer "F.Cu") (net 7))
 (segment (start 243.9135 58.001) (end 251.9115 58.001) (width 0.2) (layer "F.Cu") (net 7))
 (segment (start 251.9115 58.001) (end 252.9125 57) (width 0.2) (layer "F.Cu") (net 7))
 (segment (start 240.85676 93.876) (end 241.531 93.20176) (width 0.2) (layer "F.Cu") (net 7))
 (segment (start 234.6 58.06116) (end 234.6 58.001) (width 0.2) (layer "F.Cu") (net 7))
 (segment (start 232.9125 57) (end 233.9135 58.001) (width 0.2) (layer "F.Cu") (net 7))
 (segment (start 241.9115 58.001) (end 242.9125 57) (width 0.2) (layer "F.Cu") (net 7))
 (segment (start 241.531 77.308892) (end 243.301 75.538892) (width 0.2) (layer "F.Cu") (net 7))
 (segment (start 233.9135 58.001) (end 234.6 58.001) (width 0.2) (layer "F.Cu") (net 7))
 (segment (start 222.9125 57) (end 223.9135 58.001) (width 0.2) (layer "F.Cu") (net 7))
 (segment (start 241.531 93.20176) (end 241.531 77.308892) (width 0.2) (layer "F.Cu") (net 7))
 (segment (start 222.099 57.68516) (end 231.33094 66.9171) (width 0.2) (layer "F.Cu") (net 11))
 (segment (start 222.099 56.31484) (end 222.099 57.68516) (width 0.2) (layer "F.Cu") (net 11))
 (segment (start 248.601 51.349) (end 248.601 47.651057) (width 0.2) (layer "F.Cu") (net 11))
 (segment (start 248.601 47.651057) (end 248.248943 47.299) (width 0.2) (layer "F.Cu") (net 11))
 (segment (start 264.9125 55) (end 266.301 53.6115) (width 0.2) (layer "F.Cu") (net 11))
 (segment (start 253.2 46.75) (end 248.601 51.349) (width 0.2) (layer "F.Cu") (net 11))
 (segment (start 231.11484 47.299) (end 222.099 56.31484) (width 0.2) (layer "F.Cu") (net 11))
 (segment (start 266.301 43.1589) (end 266.0661 42.924) (width 0.2) (layer "F.Cu") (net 11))
 (segment (start 237.5171 66.9171) (end 240.38 69.78) (width 0.2) (layer "F.Cu") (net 11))
 (segment (start 248.248943 47.299) (end 231.11484 47.299) (width 0.2) (layer "F.Cu") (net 11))
 (segment (start 266.301 53.6115) (end 266.301 43.1589) (width 0.2) (layer "F.Cu") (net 11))
 (segment (start 254.51324 42.924) (end 253.2 44.23724) (width 0.2) (layer "F.Cu") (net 11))
 (segment (start 240.38 69.78) (end 240.38 92.725) (width 0.2) (layer "F.Cu") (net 11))
 (segment (start 231.33094 66.9171) (end 237.5171 66.9171) (width 0.2) (layer "F.Cu") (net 11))
 (segment (start 253.2 44.23724) (end 253.2 46.75) (width 0.2) (layer "F.Cu") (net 11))
 (segment (start 266.0661 42.924) (end 254.51324 42.924) (width 0.2) (layer "F.Cu") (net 11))
 (segment (start 247 52.95) (end 248.601 51.349) (width 0.2) (layer "F.Cu") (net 11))
 (segment (start 249.751 69.801) (end 257.2115 69.801) (width 0.2) (layer "F.Cu") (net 4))
 (segment (start 254.2 64.25) (end 252.95 63) (width 0.2) (layer "F.Cu") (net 4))
 (segment (start 222.95 63) (end 222.95 66.848) (width 0.2) (layer "F.Cu") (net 4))
 (segment (start 232 68.5) (end 230.699 67.199) (width 0.2) (layer "F.Cu") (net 4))
 (segment (start 223.301 67.199) (end 222 68.5) (width 0.2) (layer "F.Cu") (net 4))
 (segment (start 257.2115 69.801) (end 263.0625 63.95) (width 0.2) (layer "F.Cu") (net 4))
 (segment (start 246.6 59.35) (end 246.6 59.3) (width 0.2) (layer "F.Cu") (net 4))
 (segment (start 230.699 67.199) (end 223.301 67.199) (width 0.2) (layer "F.Cu") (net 4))
 (segment (start 244.75 53.3) (end 247 51.05) (width 0.2) (layer "F.Cu") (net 4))
 (segment (start 261.7125 65.3) (end 262.7625 64.25) (width 0.2) (layer "F.Cu") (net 4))
 (segment (start 262.7625 64.25) (end 254.2 64.25) (width 0.2) (layer "F.Cu") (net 4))
 (segment (start 263.0625 63.95) (end 262.7625 64.25) (width 0.2) (layer "F.Cu") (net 4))
 (segment (start 222.95 66.848) (end 223.301 67.199) (width 0.2) (layer "F.Cu") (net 4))
 (segment (start 232.95 63) (end 236.5 63) (width 0.2) (layer "F.Cu") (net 4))
 (segment (start 242.95 63) (end 249.751 69.801) (width 0.2) (layer "F.Cu") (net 4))
 (segment (start 244.3 53.3) (end 244.75 53.3) (width 0.2) (layer "F.Cu") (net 4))
 (segment (start 236.5 63) (end 242 68.5) (width 0.2) (layer "F.Cu") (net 4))
 (segment (start 259.8 65.3) (end 261.7125 65.3) (width 0.2) (layer "F.Cu") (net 4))
 (segment (start 242.95 63) (end 246.6 59.35) (width 0.2) (layer "F.Cu") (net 4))
 (via (at 246.6 59.3) (size 0.6) (drill 0.3) (layers "F.Cu" "B.Cu") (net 4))
 (via (at 259.8 65.3) (size 0.6) (drill 0.3) (layers "F.Cu" "B.Cu") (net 4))
 (via (at 244.3 53.3) (size 0.6) (drill 0.3) (layers "F.Cu" "B.Cu") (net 4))
 (segment (start 222 68.5) (end 222 75) (width 0.2) (layer "B.Cu") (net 4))
 (segment (start 252 68.5) (end 252 75) (width 0.2) (layer "B.Cu") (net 4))
 (segment (start 246.6 59.3) (end 246.6 55.6) (width 0.2) (layer "B.Cu") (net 4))
 (segment (start 246.6 55.6) (end 244.3 53.3) (width 0.2) (layer "B.Cu") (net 4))
 (segment (start 250.699 67.199) (end 252.598 65.3) (width 0.2) (layer "B.Cu") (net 4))
 (segment (start 242 68.5) (end 240.699 67.199) (width 0.2) (layer "B.Cu") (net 4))
 (segment (start 242 91.805) (end 242 75) (width 0.2) (layer "B.Cu") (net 4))
 (segment (start 259.3 65.3) (end 259.8 65.3) (width 0.2) (layer "B.Cu") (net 4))
 (segment (start 252 68.5) (end 250.699 67.199) (width 0.2) (layer "B.Cu") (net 4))
 (segment (start 250.699 67.199) (end 243.301 67.199) (width 0.2) (layer "B.Cu") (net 4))
 (segment (start 242 68.5) (end 242 75) (width 0.2) (layer "B.Cu") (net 4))
 (segment (start 243.301 67.199) (end 242 68.5) (width 0.2) (layer "B.Cu") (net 4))
 (segment (start 242.92 92.725) (end 242 91.805) (width 0.2) (layer "B.Cu") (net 4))
 (segment (start 240.699 67.199) (end 233.301 67.199) (width 0.2) (layer "B.Cu") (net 4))
 (segment (start 252.598 65.3) (end 259.3 65.3) (width 0.2) (layer "B.Cu") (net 4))
 (segment (start 233.301 67.199) (end 232 68.5) (width 0.2) (layer "B.Cu") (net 4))
 (segment (start 232 68.5) (end 232 75) (width 0.2) (layer "B.Cu") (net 4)))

